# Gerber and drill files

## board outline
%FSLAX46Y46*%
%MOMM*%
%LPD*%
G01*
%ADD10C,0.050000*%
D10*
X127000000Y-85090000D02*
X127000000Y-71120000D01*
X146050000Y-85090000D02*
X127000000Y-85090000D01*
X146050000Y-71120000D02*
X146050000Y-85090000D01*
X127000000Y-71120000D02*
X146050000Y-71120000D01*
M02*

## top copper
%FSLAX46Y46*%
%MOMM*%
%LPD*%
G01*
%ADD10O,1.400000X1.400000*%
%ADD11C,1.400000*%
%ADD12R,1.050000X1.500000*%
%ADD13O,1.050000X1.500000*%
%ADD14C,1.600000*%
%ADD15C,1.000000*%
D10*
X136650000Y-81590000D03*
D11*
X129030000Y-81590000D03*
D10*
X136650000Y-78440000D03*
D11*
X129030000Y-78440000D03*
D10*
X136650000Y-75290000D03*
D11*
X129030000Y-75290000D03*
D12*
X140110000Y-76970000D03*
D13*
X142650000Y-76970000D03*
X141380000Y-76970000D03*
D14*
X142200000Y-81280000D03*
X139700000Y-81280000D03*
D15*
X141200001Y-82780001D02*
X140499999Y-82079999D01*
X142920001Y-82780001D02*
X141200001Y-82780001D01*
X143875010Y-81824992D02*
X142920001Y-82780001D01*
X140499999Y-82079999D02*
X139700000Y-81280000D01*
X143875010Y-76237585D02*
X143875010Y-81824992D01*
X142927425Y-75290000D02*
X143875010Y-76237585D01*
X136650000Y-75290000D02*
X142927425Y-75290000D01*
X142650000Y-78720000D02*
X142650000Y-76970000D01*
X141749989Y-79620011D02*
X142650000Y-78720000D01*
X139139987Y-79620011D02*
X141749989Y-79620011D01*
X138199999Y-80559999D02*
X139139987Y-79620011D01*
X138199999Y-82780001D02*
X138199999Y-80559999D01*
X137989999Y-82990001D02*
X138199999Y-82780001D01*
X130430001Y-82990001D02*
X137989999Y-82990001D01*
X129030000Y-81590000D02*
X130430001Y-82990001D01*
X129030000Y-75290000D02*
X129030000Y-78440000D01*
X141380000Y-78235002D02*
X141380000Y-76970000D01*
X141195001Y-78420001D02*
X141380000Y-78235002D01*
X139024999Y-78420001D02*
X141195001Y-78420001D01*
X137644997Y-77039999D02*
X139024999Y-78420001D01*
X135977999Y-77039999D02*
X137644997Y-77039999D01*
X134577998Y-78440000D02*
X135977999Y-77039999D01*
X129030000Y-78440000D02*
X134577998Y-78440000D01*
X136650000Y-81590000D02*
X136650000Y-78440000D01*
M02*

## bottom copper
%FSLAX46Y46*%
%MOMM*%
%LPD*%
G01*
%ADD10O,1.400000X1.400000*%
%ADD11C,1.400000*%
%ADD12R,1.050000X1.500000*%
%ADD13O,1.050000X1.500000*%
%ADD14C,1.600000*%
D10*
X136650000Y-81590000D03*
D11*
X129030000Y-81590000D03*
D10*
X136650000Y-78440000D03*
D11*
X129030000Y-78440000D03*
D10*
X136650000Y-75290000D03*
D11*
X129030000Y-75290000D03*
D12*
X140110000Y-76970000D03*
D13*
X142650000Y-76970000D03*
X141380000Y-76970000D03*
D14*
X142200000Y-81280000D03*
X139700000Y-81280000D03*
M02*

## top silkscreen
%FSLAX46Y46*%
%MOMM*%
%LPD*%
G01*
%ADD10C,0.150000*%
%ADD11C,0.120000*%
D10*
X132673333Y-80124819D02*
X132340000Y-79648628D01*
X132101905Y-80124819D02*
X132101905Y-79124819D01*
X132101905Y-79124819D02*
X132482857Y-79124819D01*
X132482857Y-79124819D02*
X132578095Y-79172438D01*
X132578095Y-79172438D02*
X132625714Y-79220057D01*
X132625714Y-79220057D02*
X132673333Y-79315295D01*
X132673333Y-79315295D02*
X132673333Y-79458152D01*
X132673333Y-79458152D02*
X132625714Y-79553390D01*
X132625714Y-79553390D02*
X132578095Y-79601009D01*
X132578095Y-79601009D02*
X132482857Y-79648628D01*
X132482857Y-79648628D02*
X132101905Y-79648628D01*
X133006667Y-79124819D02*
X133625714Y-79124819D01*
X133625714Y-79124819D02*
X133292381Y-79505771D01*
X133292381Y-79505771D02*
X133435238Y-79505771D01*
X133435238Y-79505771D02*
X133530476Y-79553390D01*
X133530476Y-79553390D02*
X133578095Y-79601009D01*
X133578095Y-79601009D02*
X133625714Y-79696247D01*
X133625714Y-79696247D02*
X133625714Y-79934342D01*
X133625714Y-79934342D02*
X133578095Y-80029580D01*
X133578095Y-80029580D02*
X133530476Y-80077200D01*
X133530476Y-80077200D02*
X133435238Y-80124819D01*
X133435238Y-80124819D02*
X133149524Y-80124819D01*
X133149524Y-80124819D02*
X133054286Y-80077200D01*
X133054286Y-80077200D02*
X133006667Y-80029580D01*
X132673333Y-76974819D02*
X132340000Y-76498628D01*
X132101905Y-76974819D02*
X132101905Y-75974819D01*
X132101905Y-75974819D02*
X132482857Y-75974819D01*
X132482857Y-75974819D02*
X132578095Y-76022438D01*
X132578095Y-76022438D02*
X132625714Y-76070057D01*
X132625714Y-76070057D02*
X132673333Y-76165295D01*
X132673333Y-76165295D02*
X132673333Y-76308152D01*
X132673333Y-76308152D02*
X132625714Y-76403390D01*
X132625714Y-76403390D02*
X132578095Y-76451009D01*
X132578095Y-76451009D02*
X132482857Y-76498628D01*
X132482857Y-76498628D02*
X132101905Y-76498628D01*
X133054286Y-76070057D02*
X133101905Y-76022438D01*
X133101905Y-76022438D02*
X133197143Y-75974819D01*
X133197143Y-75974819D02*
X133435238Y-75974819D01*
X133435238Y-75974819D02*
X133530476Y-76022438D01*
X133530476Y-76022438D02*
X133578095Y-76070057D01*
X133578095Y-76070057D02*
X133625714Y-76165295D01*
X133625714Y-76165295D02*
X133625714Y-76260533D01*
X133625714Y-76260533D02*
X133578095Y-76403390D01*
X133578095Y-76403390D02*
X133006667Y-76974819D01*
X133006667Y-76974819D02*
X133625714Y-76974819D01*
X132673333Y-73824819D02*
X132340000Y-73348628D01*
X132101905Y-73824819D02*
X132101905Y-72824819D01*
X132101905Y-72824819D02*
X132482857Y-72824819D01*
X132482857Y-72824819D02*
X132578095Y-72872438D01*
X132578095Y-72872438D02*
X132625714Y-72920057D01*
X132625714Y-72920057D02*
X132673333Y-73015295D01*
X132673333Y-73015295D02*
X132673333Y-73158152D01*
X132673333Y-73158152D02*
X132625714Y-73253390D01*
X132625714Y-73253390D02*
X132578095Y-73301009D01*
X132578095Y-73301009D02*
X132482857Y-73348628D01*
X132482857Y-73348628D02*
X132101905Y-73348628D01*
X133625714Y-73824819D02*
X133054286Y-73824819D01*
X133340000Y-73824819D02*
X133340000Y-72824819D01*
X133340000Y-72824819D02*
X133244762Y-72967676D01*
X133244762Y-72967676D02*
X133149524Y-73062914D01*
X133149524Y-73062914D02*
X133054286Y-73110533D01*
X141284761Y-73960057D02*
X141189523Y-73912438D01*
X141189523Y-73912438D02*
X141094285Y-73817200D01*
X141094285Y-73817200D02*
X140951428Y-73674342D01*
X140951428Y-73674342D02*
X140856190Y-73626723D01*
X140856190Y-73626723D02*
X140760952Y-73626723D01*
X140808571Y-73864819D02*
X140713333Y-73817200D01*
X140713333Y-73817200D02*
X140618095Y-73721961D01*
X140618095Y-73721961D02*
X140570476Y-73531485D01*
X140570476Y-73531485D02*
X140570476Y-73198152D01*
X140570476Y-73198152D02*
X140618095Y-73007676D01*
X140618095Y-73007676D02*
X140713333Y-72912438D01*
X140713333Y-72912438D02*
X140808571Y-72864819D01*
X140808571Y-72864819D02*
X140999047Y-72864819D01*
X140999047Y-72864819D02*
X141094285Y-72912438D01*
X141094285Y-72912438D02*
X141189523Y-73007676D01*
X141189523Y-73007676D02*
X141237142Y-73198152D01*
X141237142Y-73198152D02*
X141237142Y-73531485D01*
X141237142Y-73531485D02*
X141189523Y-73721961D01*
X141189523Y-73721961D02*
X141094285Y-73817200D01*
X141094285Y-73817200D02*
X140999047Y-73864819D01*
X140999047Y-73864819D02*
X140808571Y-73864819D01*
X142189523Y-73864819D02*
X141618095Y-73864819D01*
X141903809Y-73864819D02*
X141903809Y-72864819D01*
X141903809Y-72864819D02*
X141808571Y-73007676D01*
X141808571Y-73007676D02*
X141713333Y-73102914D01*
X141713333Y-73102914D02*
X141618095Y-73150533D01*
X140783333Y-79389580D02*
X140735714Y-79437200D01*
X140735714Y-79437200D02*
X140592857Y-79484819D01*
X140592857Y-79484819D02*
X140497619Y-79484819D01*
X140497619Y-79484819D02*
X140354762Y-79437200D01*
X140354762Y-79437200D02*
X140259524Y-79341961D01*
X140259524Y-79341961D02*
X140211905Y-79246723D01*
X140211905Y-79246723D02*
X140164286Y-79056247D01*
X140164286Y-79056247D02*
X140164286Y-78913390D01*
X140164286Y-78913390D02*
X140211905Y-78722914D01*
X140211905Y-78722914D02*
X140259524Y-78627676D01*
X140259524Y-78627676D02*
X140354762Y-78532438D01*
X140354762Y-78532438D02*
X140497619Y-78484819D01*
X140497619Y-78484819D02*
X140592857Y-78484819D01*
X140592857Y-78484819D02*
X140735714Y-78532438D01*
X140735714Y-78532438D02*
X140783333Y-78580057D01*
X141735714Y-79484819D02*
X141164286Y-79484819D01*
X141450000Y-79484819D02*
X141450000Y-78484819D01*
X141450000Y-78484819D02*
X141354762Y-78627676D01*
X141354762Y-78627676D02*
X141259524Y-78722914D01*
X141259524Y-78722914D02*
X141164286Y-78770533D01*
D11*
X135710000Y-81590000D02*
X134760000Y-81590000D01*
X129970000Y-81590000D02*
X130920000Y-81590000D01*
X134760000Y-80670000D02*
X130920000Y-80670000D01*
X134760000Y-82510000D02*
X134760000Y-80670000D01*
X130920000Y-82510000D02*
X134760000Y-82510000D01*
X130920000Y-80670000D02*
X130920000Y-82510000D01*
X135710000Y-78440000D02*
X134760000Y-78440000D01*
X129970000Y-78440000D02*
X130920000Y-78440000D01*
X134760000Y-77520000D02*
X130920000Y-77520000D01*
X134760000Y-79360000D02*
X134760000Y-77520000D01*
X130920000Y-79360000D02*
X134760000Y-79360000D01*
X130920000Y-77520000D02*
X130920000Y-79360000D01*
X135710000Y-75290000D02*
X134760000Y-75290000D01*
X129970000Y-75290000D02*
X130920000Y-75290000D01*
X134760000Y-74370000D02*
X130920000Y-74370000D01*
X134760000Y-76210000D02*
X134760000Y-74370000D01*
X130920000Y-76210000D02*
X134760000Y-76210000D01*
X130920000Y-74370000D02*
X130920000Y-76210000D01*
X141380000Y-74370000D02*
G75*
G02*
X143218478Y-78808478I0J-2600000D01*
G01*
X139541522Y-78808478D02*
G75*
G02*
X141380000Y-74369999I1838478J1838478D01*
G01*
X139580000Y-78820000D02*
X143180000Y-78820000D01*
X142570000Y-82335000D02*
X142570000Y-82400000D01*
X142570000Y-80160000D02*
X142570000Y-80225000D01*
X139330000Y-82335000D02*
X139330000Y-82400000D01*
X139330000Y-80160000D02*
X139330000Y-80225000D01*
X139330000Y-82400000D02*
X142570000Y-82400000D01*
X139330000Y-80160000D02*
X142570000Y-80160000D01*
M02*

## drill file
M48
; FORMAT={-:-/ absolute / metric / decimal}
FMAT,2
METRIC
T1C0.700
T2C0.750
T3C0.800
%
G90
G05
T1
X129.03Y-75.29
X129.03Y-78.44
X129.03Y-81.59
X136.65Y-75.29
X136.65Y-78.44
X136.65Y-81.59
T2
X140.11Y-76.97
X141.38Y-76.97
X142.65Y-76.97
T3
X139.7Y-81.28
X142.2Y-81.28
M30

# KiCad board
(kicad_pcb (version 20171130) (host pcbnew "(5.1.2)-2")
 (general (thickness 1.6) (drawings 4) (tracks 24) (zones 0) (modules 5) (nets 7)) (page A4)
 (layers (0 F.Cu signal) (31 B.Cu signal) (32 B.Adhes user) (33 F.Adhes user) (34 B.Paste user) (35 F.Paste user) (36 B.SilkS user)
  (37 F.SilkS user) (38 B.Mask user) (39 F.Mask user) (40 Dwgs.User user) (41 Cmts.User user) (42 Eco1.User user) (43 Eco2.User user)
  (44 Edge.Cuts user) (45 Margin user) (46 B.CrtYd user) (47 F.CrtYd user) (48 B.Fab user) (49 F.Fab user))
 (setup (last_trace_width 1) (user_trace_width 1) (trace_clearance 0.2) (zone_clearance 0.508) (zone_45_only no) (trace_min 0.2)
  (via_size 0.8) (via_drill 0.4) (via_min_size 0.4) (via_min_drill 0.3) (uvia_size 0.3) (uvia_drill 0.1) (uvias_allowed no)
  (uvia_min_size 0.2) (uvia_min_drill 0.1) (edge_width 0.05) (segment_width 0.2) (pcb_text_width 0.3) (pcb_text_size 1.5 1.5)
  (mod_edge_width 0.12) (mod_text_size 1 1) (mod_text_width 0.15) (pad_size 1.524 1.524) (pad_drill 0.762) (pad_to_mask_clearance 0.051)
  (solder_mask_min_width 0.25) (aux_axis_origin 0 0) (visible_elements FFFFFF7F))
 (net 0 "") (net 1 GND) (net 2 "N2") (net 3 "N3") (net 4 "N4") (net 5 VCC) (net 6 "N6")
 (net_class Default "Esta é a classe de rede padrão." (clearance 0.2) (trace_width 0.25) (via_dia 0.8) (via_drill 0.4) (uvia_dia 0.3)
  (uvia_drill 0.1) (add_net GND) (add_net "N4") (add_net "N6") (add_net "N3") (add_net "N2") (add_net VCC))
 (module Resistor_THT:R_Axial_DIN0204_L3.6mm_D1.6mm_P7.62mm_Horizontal (layer F.Cu) (at 129.03 81.59)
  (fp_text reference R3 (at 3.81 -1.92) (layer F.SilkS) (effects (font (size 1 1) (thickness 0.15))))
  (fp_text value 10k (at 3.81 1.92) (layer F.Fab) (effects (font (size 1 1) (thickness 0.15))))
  (fp_line (start 6.68 0) (end 5.73 0) (layer F.SilkS) (width 0.12))
  (fp_line (start 0.94 0) (end 1.89 0) (layer F.SilkS) (width 0.12))
  (fp_line (start 5.73 -0.92) (end 1.89 -0.92) (layer F.SilkS) (width 0.12))
  (fp_line (start 5.73 0.92) (end 5.73 -0.92) (layer F.SilkS) (width 0.12))
  (fp_line (start 1.89 0.92) (end 5.73 0.92) (layer F.SilkS) (width 0.12))
  (fp_line (start 1.89 -0.92) (end 1.89 0.92) (layer F.SilkS) (width 0.12))
  (pad 2 thru_hole oval (at 7.62 0) (size 1.4 1.4) (drill 0.7) (layers *.Cu *.Mask) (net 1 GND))
  (pad 1 thru_hole circle (at 0 0) (size 1.4 1.4) (drill 0.7) (layers *.Cu *.Mask) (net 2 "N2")))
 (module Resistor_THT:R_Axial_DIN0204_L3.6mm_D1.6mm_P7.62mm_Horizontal (layer F.Cu) (at 129.03 78.44)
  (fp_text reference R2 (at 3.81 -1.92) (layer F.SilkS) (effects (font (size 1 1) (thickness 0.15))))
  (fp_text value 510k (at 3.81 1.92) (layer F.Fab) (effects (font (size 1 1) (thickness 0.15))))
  (fp_line (start 6.68 0) (end 5.73 0) (layer F.SilkS) (width 0.12))
  (fp_line (start 0.94 0) (end 1.89 0) (layer F.SilkS) (width 0.12))
  (fp_line (start 5.73 -0.92) (end 1.89 -0.92) (layer F.SilkS) (width 0.12))
  (fp_line (start 5.73 0.92) (end 5.73 -0.92) (layer F.SilkS) (width 0.12))
  (fp_line (start 1.89 0.92) (end 5.73 0.92) (layer F.SilkS) (width 0.12))
  (fp_line (start 1.89 -0.92) (end 1.89 0.92) (layer F.SilkS) (width 0.12))
  (pad 2 thru_hole oval (at 7.62 0) (size 1.4 1.4) (drill 0.7) (layers *.Cu *.Mask) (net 1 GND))
  (pad 1 thru_hole circle (at 0 0) (size 1.4 1.4) (drill 0.7) (layers *.Cu *.Mask) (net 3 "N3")))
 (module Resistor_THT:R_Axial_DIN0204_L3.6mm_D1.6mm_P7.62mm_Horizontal (layer F.Cu) (at 129.03 75.29)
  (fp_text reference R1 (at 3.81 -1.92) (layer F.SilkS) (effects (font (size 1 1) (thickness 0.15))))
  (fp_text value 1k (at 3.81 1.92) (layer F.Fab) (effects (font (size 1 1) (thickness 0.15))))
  (fp_line (start 6.68 0) (end 5.73 0) (layer F.SilkS) (width 0.12))
  (fp_line (start 0.94 0) (end 1.89 0) (layer F.SilkS) (width 0.12))
  (fp_line (start 5.73 -0.92) (end 1.89 -0.92) (layer F.SilkS) (width 0.12))
  (fp_line (start 5.73 0.92) (end 5.73 -0.92) (layer F.SilkS) (width 0.12))
  (fp_line (start 1.89 0.92) (end 5.73 0.92) (layer F.SilkS) (width 0.12))
  (fp_line (start 1.89 -0.92) (end 1.89 0.92) (layer F.SilkS) (width 0.12))
  (pad 2 thru_hole oval (at 7.62 0) (size 1.4 1.4) (drill 0.7) (layers *.Cu *.Mask) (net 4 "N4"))
  (pad 1 thru_hole circle (at 0 0) (size 1.4 1.4) (drill 0.7) (layers *.Cu *.Mask) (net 3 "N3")))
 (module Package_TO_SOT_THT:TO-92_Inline (layer F.Cu) (at 140.11 76.97)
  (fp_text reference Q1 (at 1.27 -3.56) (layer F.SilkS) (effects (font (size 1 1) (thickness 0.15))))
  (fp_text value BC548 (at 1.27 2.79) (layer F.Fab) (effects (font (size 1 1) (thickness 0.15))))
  (fp_arc (start 1.27 0) (end 1.27 -2.6) (angle 135) (layer F.SilkS) (width 0.12))
  (fp_arc (start 1.27 0) (end 1.27 -2.6) (angle -135) (layer F.SilkS) (width 0.12))
  (fp_line (start -0.53 1.85) (end 3.07 1.85) (layer F.SilkS) (width 0.12))
  (pad 1 thru_hole rect (at 0 0) (size 1.05 1.5) (drill 0.75) (layers *.Cu *.Mask) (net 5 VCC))
  (pad 3 thru_hole oval (at 2.54 0) (size 1.05 1.5) (drill 0.75) (layers *.Cu *.Mask) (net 2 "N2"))
  (pad 2 thru_hole oval (at 1.27 0) (size 1.05 1.5) (drill 0.75) (layers *.Cu *.Mask) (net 3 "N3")))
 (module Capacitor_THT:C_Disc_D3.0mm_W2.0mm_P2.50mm (layer F.Cu) (at 139.7 81.28)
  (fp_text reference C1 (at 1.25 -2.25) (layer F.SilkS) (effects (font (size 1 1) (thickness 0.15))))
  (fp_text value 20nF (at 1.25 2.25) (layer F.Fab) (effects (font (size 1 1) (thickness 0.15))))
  (fp_line (start 2.87 1.055) (end 2.87 1.12) (layer F.SilkS) (width 0.12))
  (fp_line (start 2.87 -1.12) (end 2.87 -1.055) (layer F.SilkS) (width 0.12))
  (fp_line (start -0.37 1.055) (end -0.37 1.12) (layer F.SilkS) (width 0.12))
  (fp_line (start -0.37 -1.12) (end -0.37 -1.055) (layer F.SilkS) (width 0.12))
  (fp_line (start -0.37 1.12) (end 2.87 1.12) (layer F.SilkS) (width 0.12))
  (fp_line (start -0.37 -1.12) (end 2.87 -1.12) (layer F.SilkS) (width 0.12))
  (pad 2 thru_hole circle (at 2.5 0) (size 1.6 1.6) (drill 0.8) (layers *.Cu *.Mask) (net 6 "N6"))
  (pad 1 thru_hole circle (at 0 0) (size 1.6 1.6) (drill 0.8) (layers *.Cu *.Mask) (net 4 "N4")))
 (gr_line (start 127 85.09) (end 127 71.12) (layer Edge.Cuts) (width 0.05))
 (gr_line (start 146.05 85.09) (end 127 85.09) (layer Edge.Cuts) (width 0.05))
 (gr_line (start 146.05 71.12) (end 146.05 85.09) (layer Edge.Cuts) (width 0.05))
 (gr_line (start 127 71.12) (end 146.05 71.12) (layer Edge.Cuts) (width 0.05))
 (segment (start 141.200001 82.780001) (end 140.499999 82.079999) (width 1) (layer F.Cu) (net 4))
 (segment (start 142.920001 82.780001) (end 141.200001 82.780001) (width 1) (layer F.Cu) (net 4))
 (segment (start 143.87501 81.824992) (end 142.920001 82.780001) (width 1) (layer F.Cu) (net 4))
 (segment (start 140.499999 82.079999) (end 139.7 81.28) (width 1) (layer F.Cu) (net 4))
 (segment (start 143.87501 76.237585) (end 143.87501 81.824992) (width 1) (layer F.Cu) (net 4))
 (segment (start 142.927425 75.29) (end 143.87501 76.237585) (width 1) (layer F.Cu) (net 4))
 (segment (start 136.65 75.29) (end 142.927425 75.29) (width 1) (layer F.Cu) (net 4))
 (segment (start 142.65 78.72) (end 142.65 76.97) (width 1) (layer F.Cu) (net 2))
 (segment (start 141.749989 79.620011) (end 142.65 78.72) (width 1) (layer F.Cu) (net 2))
 (segment (start 139.139987 79.620011) (end 141.749989 79.620011) (width 1) (layer F.Cu) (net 2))
 (segment (start 138.199999 80.559999) (end 139.139987 79.620011) (width 1) (layer F.Cu) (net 2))
 (segment (start 138.199999 82.780001) (end 138.199999 80.559999) (width 1) (layer F.Cu) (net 2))
 (segment (start 137.989999 82.990001) (end 138.199999 82.780001) (width 1) (layer F.Cu) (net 2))
 (segment (start 130.430001 82.990001) (end 137.989999 82.990001) (width 1) (layer F.Cu) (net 2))
 (segment (start 129.03 81.59) (end 130.430001 82.990001) (width 1) (layer F.Cu) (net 2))
 (segment (start 129.03 75.29) (end 129.03 78.44) (width 1) (layer F.Cu) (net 3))
 (segment (start 141.38 78.235002) (end 141.38 76.97) (width 1) (layer F.Cu) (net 3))
 (segment (start 141.195001 78.420001) (end 141.38 78.235002) (width 1) (layer F.Cu) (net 3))
 (segment (start 139.024999 78.420001) (end 141.195001 78.420001) (width 1) (layer F.Cu) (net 3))
 (segment (start 137.644997 77.039999) (end 139.024999 78.420001) (width 1) (layer F.Cu) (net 3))
 (segment (start 135.977999 77.039999) (end 137.644997 77.039999) (width 1) (layer F.Cu) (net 3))
 (segment (start 134.577998 78.44) (end 135.977999 77.039999) (width 1) (layer F.Cu) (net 3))
 (segment (start 129.03 78.44) (end 134.577998 78.44) (width 1) (layer F.Cu) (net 3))
 (segment (start 136.65 81.59) (end 136.65 78.44) (width 1) (layer F.Cu) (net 1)))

